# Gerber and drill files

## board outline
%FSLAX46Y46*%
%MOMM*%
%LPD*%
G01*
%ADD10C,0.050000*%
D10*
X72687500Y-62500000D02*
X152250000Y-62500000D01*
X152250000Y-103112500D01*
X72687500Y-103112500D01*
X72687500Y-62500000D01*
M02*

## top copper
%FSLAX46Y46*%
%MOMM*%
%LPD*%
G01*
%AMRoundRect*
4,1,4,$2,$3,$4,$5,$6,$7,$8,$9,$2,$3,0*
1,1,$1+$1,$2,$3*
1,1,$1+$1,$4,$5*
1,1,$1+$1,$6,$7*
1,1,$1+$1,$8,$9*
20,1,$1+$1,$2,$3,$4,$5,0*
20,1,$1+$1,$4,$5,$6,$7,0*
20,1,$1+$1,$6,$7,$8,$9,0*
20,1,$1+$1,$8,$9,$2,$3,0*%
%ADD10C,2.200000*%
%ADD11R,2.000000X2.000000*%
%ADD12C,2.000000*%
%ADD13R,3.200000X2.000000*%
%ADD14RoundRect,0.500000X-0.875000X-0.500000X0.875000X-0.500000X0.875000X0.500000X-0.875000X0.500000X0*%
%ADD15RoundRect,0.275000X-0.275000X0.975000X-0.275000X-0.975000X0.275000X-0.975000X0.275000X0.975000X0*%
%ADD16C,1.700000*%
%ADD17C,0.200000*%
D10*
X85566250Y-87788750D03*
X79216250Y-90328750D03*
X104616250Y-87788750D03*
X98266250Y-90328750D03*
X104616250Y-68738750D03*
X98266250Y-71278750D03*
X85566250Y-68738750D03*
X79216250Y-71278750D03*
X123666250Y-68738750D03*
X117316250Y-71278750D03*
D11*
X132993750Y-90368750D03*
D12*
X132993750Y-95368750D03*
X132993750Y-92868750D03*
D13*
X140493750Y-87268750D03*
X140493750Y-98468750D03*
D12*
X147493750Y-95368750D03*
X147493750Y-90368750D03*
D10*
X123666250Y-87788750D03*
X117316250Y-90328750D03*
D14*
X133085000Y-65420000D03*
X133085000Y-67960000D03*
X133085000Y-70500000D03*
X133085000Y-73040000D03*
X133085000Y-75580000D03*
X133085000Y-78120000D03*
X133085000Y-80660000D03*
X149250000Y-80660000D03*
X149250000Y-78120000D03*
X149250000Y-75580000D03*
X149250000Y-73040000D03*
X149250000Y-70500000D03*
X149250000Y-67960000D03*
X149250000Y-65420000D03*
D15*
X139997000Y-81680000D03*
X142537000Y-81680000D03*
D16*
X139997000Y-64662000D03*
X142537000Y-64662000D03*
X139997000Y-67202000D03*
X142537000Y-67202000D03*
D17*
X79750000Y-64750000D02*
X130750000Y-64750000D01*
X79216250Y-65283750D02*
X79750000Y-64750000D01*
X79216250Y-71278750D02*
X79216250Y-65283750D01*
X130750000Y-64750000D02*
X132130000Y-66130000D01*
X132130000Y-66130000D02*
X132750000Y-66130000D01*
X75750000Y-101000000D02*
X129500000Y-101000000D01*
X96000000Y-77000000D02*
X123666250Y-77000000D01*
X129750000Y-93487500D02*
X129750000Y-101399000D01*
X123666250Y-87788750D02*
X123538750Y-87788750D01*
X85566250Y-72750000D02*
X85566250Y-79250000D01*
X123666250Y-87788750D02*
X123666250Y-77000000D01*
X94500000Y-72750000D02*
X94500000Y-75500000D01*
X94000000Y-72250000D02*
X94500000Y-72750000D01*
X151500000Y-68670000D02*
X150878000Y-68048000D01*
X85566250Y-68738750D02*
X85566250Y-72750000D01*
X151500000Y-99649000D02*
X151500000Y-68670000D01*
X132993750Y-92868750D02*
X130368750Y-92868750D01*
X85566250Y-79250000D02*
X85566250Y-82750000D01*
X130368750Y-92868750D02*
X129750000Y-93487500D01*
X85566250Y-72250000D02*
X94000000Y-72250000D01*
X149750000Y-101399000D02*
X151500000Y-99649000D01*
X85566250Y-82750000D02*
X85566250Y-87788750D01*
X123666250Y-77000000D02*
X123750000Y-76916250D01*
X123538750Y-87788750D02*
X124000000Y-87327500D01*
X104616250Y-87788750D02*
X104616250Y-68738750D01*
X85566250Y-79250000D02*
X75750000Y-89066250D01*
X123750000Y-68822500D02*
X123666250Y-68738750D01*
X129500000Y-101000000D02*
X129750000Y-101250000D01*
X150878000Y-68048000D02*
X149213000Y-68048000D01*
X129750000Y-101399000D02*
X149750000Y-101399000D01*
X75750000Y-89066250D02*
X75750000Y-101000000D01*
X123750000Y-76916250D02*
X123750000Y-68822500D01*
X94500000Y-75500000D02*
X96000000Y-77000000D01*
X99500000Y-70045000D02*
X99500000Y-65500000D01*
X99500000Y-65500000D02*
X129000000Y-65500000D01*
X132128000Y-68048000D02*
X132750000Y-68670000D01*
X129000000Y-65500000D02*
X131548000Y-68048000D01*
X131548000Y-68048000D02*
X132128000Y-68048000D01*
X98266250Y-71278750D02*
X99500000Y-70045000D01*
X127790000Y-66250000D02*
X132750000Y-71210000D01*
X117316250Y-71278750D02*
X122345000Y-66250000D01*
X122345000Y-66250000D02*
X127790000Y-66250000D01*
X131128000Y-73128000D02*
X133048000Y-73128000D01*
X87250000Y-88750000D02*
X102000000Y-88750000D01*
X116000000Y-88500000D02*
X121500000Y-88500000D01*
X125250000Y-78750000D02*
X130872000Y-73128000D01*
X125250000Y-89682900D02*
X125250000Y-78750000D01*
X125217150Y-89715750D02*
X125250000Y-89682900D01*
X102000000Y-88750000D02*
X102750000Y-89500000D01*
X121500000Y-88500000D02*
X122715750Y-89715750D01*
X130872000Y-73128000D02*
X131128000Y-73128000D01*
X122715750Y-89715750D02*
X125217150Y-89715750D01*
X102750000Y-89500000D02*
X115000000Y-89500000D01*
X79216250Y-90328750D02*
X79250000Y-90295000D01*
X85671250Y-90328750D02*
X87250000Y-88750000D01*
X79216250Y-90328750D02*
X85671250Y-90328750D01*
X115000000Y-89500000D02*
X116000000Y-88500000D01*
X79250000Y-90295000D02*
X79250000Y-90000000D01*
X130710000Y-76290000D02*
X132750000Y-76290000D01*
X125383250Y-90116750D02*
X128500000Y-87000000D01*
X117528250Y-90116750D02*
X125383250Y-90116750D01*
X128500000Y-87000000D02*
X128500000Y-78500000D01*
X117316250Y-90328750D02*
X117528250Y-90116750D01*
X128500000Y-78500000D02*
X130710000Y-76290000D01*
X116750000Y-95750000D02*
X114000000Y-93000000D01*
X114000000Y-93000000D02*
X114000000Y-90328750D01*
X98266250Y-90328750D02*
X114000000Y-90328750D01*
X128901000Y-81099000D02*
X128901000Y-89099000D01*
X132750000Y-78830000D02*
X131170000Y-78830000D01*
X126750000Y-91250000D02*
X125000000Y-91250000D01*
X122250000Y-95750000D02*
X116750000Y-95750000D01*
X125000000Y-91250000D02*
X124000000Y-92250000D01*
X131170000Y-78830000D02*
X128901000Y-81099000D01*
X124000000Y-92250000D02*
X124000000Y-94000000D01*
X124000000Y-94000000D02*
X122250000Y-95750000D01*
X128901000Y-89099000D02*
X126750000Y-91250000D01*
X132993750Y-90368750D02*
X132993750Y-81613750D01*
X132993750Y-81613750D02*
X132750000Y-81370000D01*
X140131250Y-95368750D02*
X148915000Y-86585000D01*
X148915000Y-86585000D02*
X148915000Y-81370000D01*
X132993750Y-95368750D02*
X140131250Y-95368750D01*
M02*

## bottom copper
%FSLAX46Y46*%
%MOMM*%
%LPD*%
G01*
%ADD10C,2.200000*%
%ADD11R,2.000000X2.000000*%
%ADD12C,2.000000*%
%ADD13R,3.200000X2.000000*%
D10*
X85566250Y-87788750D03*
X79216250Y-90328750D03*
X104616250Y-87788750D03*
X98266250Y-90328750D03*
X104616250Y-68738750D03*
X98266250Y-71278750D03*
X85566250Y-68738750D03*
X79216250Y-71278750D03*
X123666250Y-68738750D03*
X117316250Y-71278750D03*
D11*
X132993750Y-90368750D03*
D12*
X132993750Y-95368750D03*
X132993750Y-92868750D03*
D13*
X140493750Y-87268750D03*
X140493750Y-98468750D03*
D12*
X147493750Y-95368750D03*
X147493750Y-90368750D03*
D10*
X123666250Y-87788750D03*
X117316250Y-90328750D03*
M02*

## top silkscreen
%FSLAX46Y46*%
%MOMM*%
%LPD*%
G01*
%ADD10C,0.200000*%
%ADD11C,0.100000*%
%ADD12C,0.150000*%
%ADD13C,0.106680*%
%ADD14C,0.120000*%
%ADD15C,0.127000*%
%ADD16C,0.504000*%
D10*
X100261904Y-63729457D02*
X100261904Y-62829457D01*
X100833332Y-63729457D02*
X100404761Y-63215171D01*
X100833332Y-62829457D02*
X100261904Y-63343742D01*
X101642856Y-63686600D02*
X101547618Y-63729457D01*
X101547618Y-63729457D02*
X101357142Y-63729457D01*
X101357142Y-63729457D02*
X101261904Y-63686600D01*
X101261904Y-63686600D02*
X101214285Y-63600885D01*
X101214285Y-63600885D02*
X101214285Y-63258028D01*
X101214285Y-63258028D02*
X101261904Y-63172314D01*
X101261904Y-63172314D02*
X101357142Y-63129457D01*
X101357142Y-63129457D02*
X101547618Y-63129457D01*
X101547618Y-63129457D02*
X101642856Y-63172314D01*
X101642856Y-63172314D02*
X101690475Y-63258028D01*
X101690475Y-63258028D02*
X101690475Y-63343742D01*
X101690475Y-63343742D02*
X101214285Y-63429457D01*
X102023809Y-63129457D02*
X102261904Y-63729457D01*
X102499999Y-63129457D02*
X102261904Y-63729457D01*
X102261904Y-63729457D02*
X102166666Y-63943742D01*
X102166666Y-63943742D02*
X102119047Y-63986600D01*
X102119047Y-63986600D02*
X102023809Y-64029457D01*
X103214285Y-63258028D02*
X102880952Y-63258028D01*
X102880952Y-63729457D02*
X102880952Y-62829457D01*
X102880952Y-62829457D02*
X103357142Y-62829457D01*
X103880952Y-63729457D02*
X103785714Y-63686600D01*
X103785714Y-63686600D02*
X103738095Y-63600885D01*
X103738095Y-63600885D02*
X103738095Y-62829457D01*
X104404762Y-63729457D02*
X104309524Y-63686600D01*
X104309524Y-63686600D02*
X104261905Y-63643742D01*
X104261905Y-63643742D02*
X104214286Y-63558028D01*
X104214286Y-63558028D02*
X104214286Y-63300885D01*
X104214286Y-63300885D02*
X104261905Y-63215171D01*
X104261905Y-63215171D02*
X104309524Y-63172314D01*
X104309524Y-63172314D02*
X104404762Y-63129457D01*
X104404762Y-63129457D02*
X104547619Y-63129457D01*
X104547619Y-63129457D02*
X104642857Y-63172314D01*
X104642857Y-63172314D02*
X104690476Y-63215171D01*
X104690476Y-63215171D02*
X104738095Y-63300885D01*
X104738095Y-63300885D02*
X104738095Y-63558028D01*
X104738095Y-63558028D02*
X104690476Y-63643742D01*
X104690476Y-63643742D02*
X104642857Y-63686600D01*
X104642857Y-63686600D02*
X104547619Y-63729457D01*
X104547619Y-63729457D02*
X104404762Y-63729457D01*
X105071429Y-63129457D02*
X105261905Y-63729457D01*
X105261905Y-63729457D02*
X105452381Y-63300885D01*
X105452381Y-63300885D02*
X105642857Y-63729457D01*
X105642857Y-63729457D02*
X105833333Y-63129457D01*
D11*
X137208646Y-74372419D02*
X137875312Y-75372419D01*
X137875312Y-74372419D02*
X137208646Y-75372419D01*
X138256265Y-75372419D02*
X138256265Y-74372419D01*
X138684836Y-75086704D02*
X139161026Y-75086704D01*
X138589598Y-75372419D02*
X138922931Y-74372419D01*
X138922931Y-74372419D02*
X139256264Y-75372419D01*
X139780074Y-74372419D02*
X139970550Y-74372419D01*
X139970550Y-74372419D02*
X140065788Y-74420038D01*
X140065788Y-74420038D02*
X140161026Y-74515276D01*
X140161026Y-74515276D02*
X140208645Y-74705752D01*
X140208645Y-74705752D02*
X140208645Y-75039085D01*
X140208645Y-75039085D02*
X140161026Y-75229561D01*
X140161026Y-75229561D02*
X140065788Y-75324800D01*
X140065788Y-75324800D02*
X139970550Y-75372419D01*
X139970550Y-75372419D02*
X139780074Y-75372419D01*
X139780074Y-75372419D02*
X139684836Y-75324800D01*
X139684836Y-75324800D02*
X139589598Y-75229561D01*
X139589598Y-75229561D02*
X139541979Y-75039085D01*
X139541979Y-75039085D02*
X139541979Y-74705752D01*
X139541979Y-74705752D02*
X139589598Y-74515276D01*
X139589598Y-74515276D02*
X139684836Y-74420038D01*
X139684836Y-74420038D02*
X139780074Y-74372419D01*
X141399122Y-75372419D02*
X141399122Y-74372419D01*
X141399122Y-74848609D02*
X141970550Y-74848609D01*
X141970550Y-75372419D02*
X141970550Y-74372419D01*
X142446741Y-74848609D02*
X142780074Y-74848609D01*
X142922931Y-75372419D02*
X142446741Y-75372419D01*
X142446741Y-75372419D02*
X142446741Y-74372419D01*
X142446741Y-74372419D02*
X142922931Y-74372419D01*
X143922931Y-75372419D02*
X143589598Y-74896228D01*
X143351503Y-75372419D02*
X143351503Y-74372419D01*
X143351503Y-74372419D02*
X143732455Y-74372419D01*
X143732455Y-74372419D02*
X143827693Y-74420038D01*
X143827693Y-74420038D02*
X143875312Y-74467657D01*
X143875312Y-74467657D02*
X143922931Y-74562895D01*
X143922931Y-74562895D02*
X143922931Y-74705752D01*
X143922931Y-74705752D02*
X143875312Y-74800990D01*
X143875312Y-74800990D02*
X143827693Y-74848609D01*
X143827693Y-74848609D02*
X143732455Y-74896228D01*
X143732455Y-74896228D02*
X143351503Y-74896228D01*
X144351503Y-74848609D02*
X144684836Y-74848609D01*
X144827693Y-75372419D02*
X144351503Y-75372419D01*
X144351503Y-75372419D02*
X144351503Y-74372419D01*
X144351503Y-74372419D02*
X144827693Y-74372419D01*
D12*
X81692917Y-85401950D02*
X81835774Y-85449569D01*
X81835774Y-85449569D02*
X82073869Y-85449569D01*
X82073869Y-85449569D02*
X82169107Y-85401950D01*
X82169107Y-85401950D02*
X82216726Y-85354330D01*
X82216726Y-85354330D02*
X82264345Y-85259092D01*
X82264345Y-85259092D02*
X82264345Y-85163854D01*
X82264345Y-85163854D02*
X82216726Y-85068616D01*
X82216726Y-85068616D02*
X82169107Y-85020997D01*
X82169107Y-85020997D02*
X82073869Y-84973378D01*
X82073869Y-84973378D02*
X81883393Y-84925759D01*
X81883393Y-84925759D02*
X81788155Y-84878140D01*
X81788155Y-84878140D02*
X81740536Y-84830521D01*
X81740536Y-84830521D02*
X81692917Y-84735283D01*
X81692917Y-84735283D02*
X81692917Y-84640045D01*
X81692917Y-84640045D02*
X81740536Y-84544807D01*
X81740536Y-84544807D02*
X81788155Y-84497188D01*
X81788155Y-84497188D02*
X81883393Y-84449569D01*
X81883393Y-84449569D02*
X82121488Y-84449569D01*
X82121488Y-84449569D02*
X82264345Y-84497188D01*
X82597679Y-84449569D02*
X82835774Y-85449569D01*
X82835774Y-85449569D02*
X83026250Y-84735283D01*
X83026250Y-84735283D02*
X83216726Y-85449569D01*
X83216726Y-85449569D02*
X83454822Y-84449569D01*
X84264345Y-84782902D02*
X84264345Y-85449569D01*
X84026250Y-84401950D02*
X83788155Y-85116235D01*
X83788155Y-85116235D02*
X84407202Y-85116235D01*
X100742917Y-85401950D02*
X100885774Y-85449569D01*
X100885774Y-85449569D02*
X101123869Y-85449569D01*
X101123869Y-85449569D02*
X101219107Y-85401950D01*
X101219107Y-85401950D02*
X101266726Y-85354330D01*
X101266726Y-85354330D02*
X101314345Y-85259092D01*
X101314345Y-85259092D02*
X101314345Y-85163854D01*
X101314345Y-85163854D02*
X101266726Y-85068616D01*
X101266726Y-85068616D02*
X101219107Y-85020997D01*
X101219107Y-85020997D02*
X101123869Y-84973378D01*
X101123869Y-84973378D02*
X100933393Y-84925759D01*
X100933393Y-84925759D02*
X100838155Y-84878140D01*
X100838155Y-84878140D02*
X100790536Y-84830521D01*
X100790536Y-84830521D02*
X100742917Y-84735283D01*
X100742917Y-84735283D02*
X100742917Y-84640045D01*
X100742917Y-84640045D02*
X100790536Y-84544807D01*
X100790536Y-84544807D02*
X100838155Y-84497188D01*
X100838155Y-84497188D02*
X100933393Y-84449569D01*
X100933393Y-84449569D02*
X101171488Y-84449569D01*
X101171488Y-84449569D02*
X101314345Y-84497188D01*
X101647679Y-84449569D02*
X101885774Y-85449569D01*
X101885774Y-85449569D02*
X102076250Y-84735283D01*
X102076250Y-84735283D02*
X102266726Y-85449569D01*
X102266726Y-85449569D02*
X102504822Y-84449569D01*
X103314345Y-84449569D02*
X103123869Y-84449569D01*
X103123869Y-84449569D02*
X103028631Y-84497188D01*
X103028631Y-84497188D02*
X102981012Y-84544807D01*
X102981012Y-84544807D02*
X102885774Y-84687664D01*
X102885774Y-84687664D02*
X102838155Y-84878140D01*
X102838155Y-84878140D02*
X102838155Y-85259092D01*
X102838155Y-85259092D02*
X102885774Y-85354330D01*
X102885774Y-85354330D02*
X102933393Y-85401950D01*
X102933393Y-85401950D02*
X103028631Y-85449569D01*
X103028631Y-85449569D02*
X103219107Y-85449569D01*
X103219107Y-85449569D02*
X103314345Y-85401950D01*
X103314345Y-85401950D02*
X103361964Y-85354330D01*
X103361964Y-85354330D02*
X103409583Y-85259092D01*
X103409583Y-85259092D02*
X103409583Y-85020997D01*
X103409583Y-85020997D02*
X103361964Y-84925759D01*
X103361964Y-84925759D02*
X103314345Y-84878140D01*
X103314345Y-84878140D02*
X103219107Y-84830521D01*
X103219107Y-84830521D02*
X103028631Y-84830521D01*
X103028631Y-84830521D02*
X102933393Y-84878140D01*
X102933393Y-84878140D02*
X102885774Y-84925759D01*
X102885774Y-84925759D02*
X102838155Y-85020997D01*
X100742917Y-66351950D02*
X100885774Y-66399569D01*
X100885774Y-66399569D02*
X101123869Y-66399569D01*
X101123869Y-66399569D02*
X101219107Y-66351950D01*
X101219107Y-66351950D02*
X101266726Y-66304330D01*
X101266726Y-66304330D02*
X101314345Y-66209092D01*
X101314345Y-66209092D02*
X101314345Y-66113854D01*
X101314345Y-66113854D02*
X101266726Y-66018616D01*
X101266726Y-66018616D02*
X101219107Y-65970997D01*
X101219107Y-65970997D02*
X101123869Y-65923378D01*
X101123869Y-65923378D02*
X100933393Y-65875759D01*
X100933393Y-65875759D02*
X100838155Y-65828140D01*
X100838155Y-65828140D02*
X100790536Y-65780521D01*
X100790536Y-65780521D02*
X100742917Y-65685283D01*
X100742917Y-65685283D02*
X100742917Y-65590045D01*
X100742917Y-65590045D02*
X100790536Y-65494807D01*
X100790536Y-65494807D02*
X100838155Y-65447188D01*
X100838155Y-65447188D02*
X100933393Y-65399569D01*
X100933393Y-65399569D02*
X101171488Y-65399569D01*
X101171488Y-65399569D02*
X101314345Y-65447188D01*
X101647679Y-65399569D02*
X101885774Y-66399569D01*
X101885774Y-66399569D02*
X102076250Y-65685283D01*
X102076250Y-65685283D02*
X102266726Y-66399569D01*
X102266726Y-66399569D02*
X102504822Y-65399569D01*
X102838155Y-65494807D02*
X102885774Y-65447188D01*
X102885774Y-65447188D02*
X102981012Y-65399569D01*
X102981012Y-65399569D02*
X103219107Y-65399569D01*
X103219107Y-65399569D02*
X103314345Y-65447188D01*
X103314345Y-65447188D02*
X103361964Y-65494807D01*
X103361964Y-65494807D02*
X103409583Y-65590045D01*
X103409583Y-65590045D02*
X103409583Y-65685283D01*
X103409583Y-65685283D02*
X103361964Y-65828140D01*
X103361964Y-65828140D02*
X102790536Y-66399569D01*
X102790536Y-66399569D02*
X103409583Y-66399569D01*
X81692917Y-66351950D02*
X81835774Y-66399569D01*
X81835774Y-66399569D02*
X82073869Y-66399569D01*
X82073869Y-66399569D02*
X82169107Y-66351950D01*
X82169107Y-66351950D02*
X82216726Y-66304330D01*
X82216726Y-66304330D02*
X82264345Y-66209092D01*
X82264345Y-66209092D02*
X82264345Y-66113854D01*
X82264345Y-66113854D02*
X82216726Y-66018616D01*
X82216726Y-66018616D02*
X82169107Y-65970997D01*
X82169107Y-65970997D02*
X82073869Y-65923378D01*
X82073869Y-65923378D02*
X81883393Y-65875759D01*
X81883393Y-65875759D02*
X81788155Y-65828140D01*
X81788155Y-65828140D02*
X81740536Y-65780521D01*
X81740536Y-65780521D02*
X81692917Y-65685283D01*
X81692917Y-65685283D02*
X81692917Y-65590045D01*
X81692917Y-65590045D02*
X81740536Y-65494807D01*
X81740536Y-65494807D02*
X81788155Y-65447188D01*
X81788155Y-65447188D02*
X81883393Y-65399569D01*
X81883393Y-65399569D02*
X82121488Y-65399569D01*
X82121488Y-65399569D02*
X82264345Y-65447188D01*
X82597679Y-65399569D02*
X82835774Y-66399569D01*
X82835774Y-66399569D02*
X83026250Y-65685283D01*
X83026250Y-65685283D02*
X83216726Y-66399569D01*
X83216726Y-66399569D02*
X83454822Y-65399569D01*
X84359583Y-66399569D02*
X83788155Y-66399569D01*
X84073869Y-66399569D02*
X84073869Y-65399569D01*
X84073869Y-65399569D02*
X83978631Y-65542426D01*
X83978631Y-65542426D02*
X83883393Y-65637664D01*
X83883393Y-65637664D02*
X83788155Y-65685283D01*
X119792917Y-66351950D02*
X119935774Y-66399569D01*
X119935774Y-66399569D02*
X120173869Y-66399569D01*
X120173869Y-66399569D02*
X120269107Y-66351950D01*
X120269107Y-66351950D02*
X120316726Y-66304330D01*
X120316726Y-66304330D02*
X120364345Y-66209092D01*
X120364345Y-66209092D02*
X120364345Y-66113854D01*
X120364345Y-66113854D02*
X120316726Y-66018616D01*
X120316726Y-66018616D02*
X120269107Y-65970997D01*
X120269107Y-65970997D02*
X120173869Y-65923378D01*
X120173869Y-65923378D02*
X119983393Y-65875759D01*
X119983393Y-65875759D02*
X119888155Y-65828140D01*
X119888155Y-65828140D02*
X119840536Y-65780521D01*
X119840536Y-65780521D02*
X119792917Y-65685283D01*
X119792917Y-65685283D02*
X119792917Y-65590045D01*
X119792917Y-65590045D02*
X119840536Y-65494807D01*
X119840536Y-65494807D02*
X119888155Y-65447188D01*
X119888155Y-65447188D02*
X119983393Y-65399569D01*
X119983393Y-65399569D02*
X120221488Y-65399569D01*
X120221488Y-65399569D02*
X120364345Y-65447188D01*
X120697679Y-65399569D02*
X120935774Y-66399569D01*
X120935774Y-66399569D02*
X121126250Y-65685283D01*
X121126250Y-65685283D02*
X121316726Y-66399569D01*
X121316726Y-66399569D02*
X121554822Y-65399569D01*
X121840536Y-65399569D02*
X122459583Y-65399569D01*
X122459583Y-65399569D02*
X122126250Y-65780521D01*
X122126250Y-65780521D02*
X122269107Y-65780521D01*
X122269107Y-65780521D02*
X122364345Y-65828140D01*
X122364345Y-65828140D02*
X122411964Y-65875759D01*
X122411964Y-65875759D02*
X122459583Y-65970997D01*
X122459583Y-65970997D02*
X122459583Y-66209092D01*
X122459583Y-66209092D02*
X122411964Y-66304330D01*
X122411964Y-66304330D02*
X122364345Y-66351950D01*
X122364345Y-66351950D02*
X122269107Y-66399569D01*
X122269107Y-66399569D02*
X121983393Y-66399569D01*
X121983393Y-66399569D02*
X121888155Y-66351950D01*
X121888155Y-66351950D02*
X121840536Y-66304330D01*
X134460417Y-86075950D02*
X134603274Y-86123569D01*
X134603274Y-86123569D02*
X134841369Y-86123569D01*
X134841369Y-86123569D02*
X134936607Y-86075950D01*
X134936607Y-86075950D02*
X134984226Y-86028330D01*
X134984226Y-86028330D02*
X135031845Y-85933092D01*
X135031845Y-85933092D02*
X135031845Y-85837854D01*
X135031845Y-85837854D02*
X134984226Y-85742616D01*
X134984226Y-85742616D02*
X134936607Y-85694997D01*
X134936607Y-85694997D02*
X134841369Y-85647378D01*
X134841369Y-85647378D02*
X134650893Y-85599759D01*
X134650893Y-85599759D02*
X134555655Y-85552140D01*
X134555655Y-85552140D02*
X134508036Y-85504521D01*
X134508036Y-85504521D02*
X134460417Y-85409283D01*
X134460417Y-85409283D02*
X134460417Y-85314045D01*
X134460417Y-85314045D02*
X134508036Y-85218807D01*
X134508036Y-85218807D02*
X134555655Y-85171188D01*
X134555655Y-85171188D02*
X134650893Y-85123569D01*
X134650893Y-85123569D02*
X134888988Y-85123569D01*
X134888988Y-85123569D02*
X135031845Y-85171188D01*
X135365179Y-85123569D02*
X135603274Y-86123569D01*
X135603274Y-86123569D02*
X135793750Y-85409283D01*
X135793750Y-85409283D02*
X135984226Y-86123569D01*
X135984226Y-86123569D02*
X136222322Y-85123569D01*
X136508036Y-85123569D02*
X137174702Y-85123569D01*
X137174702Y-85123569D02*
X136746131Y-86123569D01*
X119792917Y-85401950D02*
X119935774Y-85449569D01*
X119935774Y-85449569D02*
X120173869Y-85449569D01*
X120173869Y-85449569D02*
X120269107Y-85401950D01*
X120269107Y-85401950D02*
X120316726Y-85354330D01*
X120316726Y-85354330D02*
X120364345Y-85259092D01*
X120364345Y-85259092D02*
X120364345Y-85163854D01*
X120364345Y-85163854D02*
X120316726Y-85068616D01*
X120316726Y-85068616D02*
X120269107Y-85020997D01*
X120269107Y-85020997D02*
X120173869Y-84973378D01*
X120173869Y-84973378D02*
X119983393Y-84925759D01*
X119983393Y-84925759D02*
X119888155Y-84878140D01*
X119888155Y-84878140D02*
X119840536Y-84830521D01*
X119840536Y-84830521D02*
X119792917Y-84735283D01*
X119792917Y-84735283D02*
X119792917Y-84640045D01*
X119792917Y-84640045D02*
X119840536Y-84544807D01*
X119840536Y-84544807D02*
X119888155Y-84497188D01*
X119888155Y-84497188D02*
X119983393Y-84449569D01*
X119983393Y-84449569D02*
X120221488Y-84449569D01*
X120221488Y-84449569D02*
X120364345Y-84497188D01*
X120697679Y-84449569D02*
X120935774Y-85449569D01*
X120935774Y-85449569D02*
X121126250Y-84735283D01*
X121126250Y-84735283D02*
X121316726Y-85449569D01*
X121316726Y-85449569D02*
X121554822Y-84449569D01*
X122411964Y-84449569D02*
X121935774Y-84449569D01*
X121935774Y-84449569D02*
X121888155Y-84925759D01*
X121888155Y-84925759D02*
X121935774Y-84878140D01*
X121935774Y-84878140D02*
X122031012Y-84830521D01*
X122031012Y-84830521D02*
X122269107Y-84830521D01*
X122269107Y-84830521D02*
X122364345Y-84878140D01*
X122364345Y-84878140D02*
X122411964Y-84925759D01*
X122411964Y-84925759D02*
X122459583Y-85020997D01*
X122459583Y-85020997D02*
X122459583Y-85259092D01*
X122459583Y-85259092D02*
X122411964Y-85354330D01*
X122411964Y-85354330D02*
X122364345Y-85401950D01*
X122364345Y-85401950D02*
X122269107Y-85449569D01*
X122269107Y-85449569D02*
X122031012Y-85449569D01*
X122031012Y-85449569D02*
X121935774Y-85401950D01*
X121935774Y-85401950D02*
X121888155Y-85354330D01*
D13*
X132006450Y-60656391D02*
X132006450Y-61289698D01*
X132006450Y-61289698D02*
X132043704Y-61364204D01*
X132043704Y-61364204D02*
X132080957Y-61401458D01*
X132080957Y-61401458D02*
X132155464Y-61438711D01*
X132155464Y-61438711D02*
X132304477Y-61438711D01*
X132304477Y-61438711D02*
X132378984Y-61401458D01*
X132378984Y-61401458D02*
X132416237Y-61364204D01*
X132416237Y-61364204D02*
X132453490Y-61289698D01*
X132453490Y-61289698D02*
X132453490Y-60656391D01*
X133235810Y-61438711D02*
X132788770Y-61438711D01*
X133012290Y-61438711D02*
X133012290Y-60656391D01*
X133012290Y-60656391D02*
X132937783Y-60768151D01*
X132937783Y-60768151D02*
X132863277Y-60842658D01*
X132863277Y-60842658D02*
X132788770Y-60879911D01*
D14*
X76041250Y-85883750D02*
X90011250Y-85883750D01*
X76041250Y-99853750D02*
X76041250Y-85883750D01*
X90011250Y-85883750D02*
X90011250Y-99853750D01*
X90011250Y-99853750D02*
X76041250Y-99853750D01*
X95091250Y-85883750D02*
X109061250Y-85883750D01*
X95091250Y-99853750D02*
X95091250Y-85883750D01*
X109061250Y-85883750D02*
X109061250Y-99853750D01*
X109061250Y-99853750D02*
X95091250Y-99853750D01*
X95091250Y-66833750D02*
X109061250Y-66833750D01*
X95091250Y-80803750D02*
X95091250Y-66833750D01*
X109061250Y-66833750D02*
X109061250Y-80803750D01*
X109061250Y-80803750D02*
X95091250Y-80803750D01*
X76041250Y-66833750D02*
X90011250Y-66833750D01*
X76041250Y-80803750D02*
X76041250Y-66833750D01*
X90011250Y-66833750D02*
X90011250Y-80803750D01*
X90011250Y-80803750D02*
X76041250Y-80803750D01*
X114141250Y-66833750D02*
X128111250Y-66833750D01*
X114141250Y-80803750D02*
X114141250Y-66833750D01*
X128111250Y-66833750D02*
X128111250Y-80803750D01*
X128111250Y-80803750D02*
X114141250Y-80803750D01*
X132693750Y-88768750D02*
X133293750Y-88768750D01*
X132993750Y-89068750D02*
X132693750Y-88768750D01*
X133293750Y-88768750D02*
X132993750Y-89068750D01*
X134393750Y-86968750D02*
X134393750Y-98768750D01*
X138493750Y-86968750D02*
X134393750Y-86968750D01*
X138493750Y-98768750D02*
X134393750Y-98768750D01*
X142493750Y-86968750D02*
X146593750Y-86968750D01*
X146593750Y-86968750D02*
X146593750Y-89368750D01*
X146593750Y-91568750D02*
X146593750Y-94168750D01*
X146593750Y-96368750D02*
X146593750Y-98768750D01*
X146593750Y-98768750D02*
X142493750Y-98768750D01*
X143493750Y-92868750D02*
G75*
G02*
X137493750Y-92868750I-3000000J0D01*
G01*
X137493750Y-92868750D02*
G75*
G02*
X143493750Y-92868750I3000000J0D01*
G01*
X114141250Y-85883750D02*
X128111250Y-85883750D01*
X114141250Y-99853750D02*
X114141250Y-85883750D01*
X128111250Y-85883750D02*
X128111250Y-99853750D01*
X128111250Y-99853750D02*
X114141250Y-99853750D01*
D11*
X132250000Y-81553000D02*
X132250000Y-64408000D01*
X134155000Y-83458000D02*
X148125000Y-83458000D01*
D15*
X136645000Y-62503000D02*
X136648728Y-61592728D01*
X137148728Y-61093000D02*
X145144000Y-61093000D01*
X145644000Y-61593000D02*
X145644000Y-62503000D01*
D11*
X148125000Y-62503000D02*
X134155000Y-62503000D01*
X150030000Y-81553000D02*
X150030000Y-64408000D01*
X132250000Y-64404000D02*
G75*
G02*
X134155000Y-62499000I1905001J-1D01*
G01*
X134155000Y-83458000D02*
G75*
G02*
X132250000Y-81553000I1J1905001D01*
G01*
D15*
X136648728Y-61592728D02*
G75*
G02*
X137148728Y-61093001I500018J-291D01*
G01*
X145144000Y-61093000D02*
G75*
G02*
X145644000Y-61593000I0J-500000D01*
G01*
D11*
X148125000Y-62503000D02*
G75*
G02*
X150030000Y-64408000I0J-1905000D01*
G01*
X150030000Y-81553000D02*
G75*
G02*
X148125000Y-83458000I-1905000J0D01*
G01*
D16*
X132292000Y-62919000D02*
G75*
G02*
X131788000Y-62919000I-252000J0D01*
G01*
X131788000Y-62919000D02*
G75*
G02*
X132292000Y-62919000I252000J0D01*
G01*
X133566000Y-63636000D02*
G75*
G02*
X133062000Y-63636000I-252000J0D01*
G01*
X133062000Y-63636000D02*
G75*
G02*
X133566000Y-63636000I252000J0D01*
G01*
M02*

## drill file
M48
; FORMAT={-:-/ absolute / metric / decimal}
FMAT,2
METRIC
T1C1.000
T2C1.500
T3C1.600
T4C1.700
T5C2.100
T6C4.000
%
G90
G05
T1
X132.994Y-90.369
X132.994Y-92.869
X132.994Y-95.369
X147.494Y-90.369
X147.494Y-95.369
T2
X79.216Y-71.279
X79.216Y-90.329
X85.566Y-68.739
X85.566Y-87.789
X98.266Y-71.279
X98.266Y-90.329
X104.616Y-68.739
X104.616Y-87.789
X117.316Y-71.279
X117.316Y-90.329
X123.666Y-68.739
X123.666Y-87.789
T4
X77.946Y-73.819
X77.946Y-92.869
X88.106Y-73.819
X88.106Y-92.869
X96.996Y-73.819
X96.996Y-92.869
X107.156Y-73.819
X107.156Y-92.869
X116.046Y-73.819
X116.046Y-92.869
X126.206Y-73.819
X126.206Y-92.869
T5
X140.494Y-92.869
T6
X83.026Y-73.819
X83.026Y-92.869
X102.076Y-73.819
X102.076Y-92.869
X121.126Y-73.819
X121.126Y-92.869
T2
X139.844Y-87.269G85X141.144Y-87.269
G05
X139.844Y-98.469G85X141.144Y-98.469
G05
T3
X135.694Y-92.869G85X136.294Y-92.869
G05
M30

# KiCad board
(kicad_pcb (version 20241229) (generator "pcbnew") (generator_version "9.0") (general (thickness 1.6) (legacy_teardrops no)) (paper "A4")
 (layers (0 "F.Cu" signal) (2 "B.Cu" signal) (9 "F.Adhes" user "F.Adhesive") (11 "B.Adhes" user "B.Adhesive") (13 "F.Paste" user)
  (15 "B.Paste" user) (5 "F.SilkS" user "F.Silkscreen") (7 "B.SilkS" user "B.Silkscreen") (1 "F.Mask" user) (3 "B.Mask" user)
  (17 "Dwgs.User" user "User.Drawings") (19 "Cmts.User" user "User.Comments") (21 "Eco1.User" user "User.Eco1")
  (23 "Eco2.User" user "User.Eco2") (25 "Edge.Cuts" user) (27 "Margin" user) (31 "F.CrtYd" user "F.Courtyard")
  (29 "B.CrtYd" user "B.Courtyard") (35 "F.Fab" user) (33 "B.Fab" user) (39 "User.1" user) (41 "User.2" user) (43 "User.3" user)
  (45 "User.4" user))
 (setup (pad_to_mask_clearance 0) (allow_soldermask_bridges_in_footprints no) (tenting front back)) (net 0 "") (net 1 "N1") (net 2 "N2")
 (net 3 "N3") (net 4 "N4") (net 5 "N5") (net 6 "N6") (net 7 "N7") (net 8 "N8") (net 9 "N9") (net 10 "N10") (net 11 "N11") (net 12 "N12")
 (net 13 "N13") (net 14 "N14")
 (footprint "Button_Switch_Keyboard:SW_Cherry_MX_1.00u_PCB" (layer "F.Cu") (at 85.56625 87.78875)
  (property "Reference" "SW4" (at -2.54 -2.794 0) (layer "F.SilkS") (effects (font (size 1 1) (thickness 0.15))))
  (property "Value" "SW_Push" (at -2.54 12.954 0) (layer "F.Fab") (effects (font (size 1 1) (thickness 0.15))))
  (fp_line (start -9.525 -1.905) (end 4.445 -1.905) (stroke (width 0.12) (type solid)) (layer "F.SilkS"))
  (fp_line (start -9.525 12.065) (end -9.525 -1.905) (stroke (width 0.12) (type solid)) (layer "F.SilkS"))
  (fp_line (start 4.445 -1.905) (end 4.445 12.065) (stroke (width 0.12) (type solid)) (layer "F.SilkS"))
  (fp_line (start 4.445 12.065) (end -9.525 12.065) (stroke (width 0.12) (type solid)) (layer "F.SilkS"))
  (pad "" np_thru_hole circle (at -7.62 5.08) (size 1.7 1.7) (drill 1.7) (layers "*.Cu" "*.Mask"))
  (pad "" np_thru_hole circle (at -2.54 5.08) (size 4 4) (drill 4) (layers "*.Cu" "*.Mask"))
  (pad "" np_thru_hole circle (at 2.54 5.08) (size 1.7 1.7) (drill 1.7) (layers "*.Cu" "*.Mask"))
  (pad "1" thru_hole circle (at 0 0) (size 2.2 2.2) (drill 1.5) (layers "*.Cu" "*.Mask") (remove_unused_layers no) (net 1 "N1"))
  (pad "2" thru_hole circle (at -6.35 2.54) (size 2.2 2.2) (drill 1.5) (layers "*.Cu" "*.Mask") (remove_unused_layers no) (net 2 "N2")))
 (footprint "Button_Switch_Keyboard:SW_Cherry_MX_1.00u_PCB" (layer "F.Cu") (at 104.61625 87.78875)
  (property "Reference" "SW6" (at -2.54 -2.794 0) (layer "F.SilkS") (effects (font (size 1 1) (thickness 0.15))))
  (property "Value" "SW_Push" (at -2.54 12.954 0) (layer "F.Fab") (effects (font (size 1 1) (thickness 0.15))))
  (fp_line (start -9.525 -1.905) (end 4.445 -1.905) (stroke (width 0.12) (type solid)) (layer "F.SilkS"))
  (fp_line (start -9.525 12.065) (end -9.525 -1.905) (stroke (width 0.12) (type solid)) (layer "F.SilkS"))
  (fp_line (start 4.445 -1.905) (end 4.445 12.065) (stroke (width 0.12) (type solid)) (layer "F.SilkS"))
  (fp_line (start 4.445 12.065) (end -9.525 12.065) (stroke (width 0.12) (type solid)) (layer "F.SilkS"))
  (pad "" np_thru_hole circle (at -7.62 5.08) (size 1.7 1.7) (drill 1.7) (layers "*.Cu" "*.Mask"))
  (pad "" np_thru_hole circle (at -2.54 5.08) (size 4 4) (drill 4) (layers "*.Cu" "*.Mask"))
  (pad "" np_thru_hole circle (at 2.54 5.08) (size 1.7 1.7) (drill 1.7) (layers "*.Cu" "*.Mask"))
  (pad "1" thru_hole circle (at 0 0) (size 2.2 2.2) (drill 1.5) (layers "*.Cu" "*.Mask") (remove_unused_layers no) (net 1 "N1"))
  (pad "2" thru_hole circle (at -6.35 2.54) (size 2.2 2.2) (drill 1.5) (layers "*.Cu" "*.Mask") (remove_unused_layers no) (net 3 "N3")))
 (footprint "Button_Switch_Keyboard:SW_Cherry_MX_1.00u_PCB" (layer "F.Cu") (at 104.61625 68.73875)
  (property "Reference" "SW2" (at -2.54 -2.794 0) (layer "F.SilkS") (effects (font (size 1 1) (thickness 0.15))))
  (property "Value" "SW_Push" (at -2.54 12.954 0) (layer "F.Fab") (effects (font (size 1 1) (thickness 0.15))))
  (fp_line (start -9.525 -1.905) (end 4.445 -1.905) (stroke (width 0.12) (type solid)) (layer "F.SilkS"))
  (fp_line (start -9.525 12.065) (end -9.525 -1.905) (stroke (width 0.12) (type solid)) (layer "F.SilkS"))
  (fp_line (start 4.445 -1.905) (end 4.445 12.065) (stroke (width 0.12) (type solid)) (layer "F.SilkS"))
  (fp_line (start 4.445 12.065) (end -9.525 12.065) (stroke (width 0.12) (type solid)) (layer "F.SilkS"))
  (pad "" np_thru_hole circle (at -7.62 5.08) (size 1.7 1.7) (drill 1.7) (layers "*.Cu" "*.Mask"))
  (pad "" np_thru_hole circle (at -2.54 5.08) (size 4 4) (drill 4) (layers "*.Cu" "*.Mask"))
  (pad "" np_thru_hole circle (at 2.54 5.08) (size 1.7 1.7) (drill 1.7) (layers "*.Cu" "*.Mask"))
  (pad "1" thru_hole circle (at 0 0) (size 2.2 2.2) (drill 1.5) (layers "*.Cu" "*.Mask") (remove_unused_layers no) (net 1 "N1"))
  (pad "2" thru_hole circle (at -6.35 2.54) (size 2.2 2.2) (drill 1.5) (layers "*.Cu" "*.Mask") (remove_unused_layers no) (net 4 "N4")))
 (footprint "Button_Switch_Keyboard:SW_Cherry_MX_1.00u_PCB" (layer "F.Cu") (at 85.56625 68.73875)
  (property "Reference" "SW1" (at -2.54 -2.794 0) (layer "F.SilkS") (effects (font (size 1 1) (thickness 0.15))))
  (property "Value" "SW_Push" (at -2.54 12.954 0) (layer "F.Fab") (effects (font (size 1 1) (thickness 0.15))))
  (fp_line (start -9.525 -1.905) (end 4.445 -1.905) (stroke (width 0.12) (type solid)) (layer "F.SilkS"))
  (fp_line (start -9.525 12.065) (end -9.525 -1.905) (stroke (width 0.12) (type solid)) (layer "F.SilkS"))
  (fp_line (start 4.445 -1.905) (end 4.445 12.065) (stroke (width 0.12) (type solid)) (layer "F.SilkS"))
  (fp_line (start 4.445 12.065) (end -9.525 12.065) (stroke (width 0.12) (type solid)) (layer "F.SilkS"))
  (pad "" np_thru_hole circle (at -7.62 5.08) (size 1.7 1.7) (drill 1.7) (layers "*.Cu" "*.Mask"))
  (pad "" np_thru_hole circle (at -2.54 5.08) (size 4 4) (drill 4) (layers "*.Cu" "*.Mask"))
  (pad "" np_thru_hole circle (at 2.54 5.08) (size 1.7 1.7) (drill 1.7) (layers "*.Cu" "*.Mask"))
  (pad "1" thru_hole circle (at 0 0) (size 2.2 2.2) (drill 1.5) (layers "*.Cu" "*.Mask") (remove_unused_layers no) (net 1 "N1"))
  (pad "2" thru_hole circle (at -6.35 2.54) (size 2.2 2.2) (drill 1.5) (layers "*.Cu" "*.Mask") (remove_unused_layers no) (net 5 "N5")))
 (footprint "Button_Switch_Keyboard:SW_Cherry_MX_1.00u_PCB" (layer "F.Cu") (at 123.66625 68.73875)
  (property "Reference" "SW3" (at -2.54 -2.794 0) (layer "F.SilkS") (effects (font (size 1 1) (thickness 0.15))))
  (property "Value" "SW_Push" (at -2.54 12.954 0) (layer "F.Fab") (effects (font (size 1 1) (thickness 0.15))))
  (fp_line (start -9.525 -1.905) (end 4.445 -1.905) (stroke (width 0.12) (type solid)) (layer "F.SilkS"))
  (fp_line (start -9.525 12.065) (end -9.525 -1.905) (stroke (width 0.12) (type solid)) (layer "F.SilkS"))
  (fp_line (start 4.445 -1.905) (end 4.445 12.065) (stroke (width 0.12) (type solid)) (layer "F.SilkS"))
  (fp_line (start 4.445 12.065) (end -9.525 12.065) (stroke (width 0.12) (type solid)) (layer "F.SilkS"))
  (pad "" np_thru_hole circle (at -7.62 5.08) (size 1.7 1.7) (drill 1.7) (layers "*.Cu" "*.Mask"))
  (pad "" np_thru_hole circle (at -2.54 5.08) (size 4 4) (drill 4) (layers "*.Cu" "*.Mask"))
  (pad "" np_thru_hole circle (at 2.54 5.08) (size 1.7 1.7) (drill 1.7) (layers "*.Cu" "*.Mask"))
  (pad "1" thru_hole circle (at 0 0) (size 2.2 2.2) (drill 1.5) (layers "*.Cu" "*.Mask") (remove_unused_layers no) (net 1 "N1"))
  (pad "2" thru_hole circle (at -6.35 2.54) (size 2.2 2.2) (drill 1.5) (layers "*.Cu" "*.Mask") (remove_unused_layers no) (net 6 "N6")))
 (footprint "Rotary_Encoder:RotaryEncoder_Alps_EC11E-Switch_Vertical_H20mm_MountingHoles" (layer "F.Cu") (at 132.99375 90.36875)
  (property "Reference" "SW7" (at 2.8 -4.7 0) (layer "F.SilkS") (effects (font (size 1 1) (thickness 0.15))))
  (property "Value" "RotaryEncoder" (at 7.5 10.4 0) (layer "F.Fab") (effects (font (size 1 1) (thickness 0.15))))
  (fp_line (start -0.3 -1.6) (end 0.3 -1.6) (stroke (width 0.12) (type solid)) (layer "F.SilkS"))
  (fp_line (start 0 -1.3) (end -0.3 -1.6) (stroke (width 0.12) (type solid)) (layer "F.SilkS"))
  (fp_line (start 0.3 -1.6) (end 0 -1.3) (stroke (width 0.12) (type solid)) (layer "F.SilkS"))
  (fp_line (start 1.4 -3.4) (end 1.4 8.4) (stroke (width 0.12) (type solid)) (layer "F.SilkS"))
  (fp_line (start 5.5 -3.4) (end 1.4 -3.4) (stroke (width 0.12) (type solid)) (layer "F.SilkS"))
  (fp_line (start 5.5 8.4) (end 1.4 8.4) (stroke (width 0.12) (type solid)) (layer "F.SilkS"))
  (fp_line (start 9.5 -3.4) (end 13.6 -3.4) (stroke (width 0.12) (type solid)) (layer "F.SilkS"))
  (fp_line (start 13.6 -3.4) (end 13.6 -1) (stroke (width 0.12) (type solid)) (layer "F.SilkS"))
  (fp_line (start 13.6 1.2) (end 13.6 3.8) (stroke (width 0.12) (type solid)) (layer "F.SilkS"))
  (fp_line (start 13.6 6) (end 13.6 8.4) (stroke (width 0.12) (type solid)) (layer "F.SilkS"))
  (fp_line (start 13.6 8.4) (end 9.5 8.4) (stroke (width 0.12) (type solid)) (layer "F.SilkS"))
  (fp_circle (center 7.5 2.5) (end 10.5 2.5) (stroke (width 0.12) (type solid)) (fill no) (layer "F.SilkS"))
  (pad "" np_thru_hole oval (at 3 2.5) (size 2.2 1.6) (drill oval 2.2 1.6) (layers "*.Mask"))
  (pad "" np_thru_hole circle (at 7.5 2.5) (size 2.1 2.1) (drill 2.1) (layers "*.Mask"))
  (pad "A" thru_hole rect (at 0 0) (size 2 2) (drill 1) (layers "*.Cu" "*.Mask") (remove_unused_layers no) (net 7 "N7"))
  (pad "B" thru_hole circle (at 0 5) (size 2 2) (drill 1) (layers "*.Cu" "*.Mask") (remove_unused_layers no) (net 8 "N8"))
  (pad "C" thru_hole circle (at 0 2.5) (size 2 2) (drill 1) (layers "*.Cu" "*.Mask") (remove_unused_layers no) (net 1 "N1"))
  (pad "MP" thru_hole rect (at 7.5 -3.1) (size 3.2 2) (drill oval 2.8 1.5) (layers "*.Cu" "*.Mask") (remove_unused_layers no))
  (pad "MP" thru_hole rect (at 7.5 8.1) (size 3.2 2) (drill oval 2.8 1.5) (layers "*.Cu" "*.Mask") (remove_unused_layers no))
  (pad "S1" thru_hole circle (at 14.5 5) (size 2 2) (drill 1) (layers "*.Cu" "*.Mask") (remove_unused_layers no))
  (pad "S2" thru_hole circle (at 14.5 0) (size 2 2) (drill 1) (layers "*.Cu" "*.Mask") (remove_unused_layers no)))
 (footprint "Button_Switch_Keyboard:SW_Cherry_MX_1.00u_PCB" (layer "F.Cu") (at 123.66625 87.78875)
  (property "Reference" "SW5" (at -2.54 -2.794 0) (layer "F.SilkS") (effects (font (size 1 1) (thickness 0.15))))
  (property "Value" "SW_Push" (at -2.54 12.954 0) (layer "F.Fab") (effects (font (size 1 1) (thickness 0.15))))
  (fp_line (start -9.525 -1.905) (end 4.445 -1.905) (stroke (width 0.12) (type solid)) (layer "F.SilkS"))
  (fp_line (start -9.525 12.065) (end -9.525 -1.905) (stroke (width 0.12) (type solid)) (layer "F.SilkS"))
  (fp_line (start 4.445 -1.905) (end 4.445 12.065) (stroke (width 0.12) (type solid)) (layer "F.SilkS"))
  (fp_line (start 4.445 12.065) (end -9.525 12.065) (stroke (width 0.12) (type solid)) (layer "F.SilkS"))
  (pad "" np_thru_hole circle (at -7.62 5.08) (size 1.7 1.7) (drill 1.7) (layers "*.Cu" "*.Mask"))
  (pad "" np_thru_hole circle (at -2.54 5.08) (size 4 4) (drill 4) (layers "*.Cu" "*.Mask"))
  (pad "" np_thru_hole circle (at 2.54 5.08) (size 1.7 1.7) (drill 1.7) (layers "*.Cu" "*.Mask"))
  (pad "1" thru_hole circle (at 0 0) (size 2.2 2.2) (drill 1.5) (layers "*.Cu" "*.Mask") (remove_unused_layers no) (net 1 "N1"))
  (pad "2" thru_hole circle (at -6.35 2.54) (size 2.2 2.2) (drill 1.5) (layers "*.Cu" "*.Mask") (remove_unused_layers no) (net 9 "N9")))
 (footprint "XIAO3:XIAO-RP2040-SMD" (layer "F.Cu") (at 141.085 73.04)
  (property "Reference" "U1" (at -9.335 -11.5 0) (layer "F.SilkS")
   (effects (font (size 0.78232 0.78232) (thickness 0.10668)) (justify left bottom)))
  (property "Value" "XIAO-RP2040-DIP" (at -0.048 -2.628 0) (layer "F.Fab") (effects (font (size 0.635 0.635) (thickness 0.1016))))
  (fp_line (start -8.835 8.513) (end -8.835 -8.632) (stroke (width 0.1) (type solid)) (layer "F.SilkS"))
  (fp_line (start -6.93 10.418) (end 7.04 10.418) (stroke (width 0.1) (type solid)) (layer "F.SilkS"))
  (fp_line (start -4.44 -10.537) (end -4.436272 -11.447272) (stroke (width 0.127) (type solid)) (layer "F.SilkS"))
  (fp_line (start -3.936272 -11.947) (end 4.059 -11.947) (stroke (width 0.127) (type solid)) (layer "F.SilkS"))
  (fp_line (start 4.559 -11.447) (end 4.559 -10.537) (stroke (width 0.127) (type solid)) (layer "F.SilkS"))
  (fp_line (start 7.04 -10.537) (end -6.93 -10.537) (stroke (width 0.1) (type solid)) (layer "F.SilkS"))
  (fp_line (start 8.945 8.513) (end 8.945 -8.632) (stroke (width 0.1) (type solid)) (layer "F.SilkS"))
  (fp_arc (start -8.835 -8.636) (mid -8.277038 -9.983038) (end -6.93 -10.541) (stroke (width 0.1) (type solid)) (layer "F.SilkS"))
  (fp_arc (start -6.93 10.418) (mid -8.277038 9.860038) (end -8.835 8.513) (stroke (width 0.1) (type solid)) (layer "F.SilkS"))
  (fp_arc (start -4.436272 -11.447272) (mid -4.289724 -11.800644) (end -3.936272 -11.947) (stroke (width 0.127) (type default))
   (layer "F.SilkS"))
  (fp_arc (start 4.059 -11.947) (mid 4.412553 -11.800553) (end 4.559 -11.447) (stroke (width 0.127) (type default)) (layer "F.SilkS"))
  (fp_arc (start 7.04 -10.537) (mid 8.387038 -9.979038) (end 8.945 -8.632) (stroke (width 0.1) (type solid)) (layer "F.SilkS"))
  (fp_arc (start 8.945 8.513) (mid 8.387038 9.860038) (end 7.04 10.418) (stroke (width 0.1) (type solid)) (layer "F.SilkS"))
  (fp_circle (center -9.045 -10.121) (end -9.045 -10.375) (stroke (width 0.5) (type solid)) (fill yes) (layer "F.SilkS"))
  (fp_circle (center -7.771 -9.404) (end -7.771 -9.658) (stroke (width 0.5) (type solid)) (fill yes) (layer "F.SilkS"))
  (pad "1" smd roundrect (at -8 -7.62) (size 2.75 2) (layers "F.Cu" "F.Mask" "F.Paste") (roundrect_rratio 0.25) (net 5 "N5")
   (solder_mask_margin 0.0508) (thermal_bridge_angle 45))
  (pad "2" smd roundrect (at -8 -5.08) (size 2.75 2) (layers "F.Cu" "F.Mask" "F.Paste") (roundrect_rratio 0.25) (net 4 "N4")
   (solder_mask_margin 0.0508) (thermal_bridge_angle 45))
  (pad "3" smd roundrect (at -8 -2.54) (size 2.75 2) (layers "F.Cu" "F.Mask" "F.Paste") (roundrect_rratio 0.25) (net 6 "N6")
   (solder_mask_margin 0.0508) (thermal_bridge_angle 45))
  (pad "4" smd roundrect (at -8 0) (size 2.75 2) (layers "F.Cu" "F.Mask" "F.Paste") (roundrect_rratio 0.25) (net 2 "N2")
   (solder_mask_margin 0.0508) (thermal_bridge_angle 45))
  (pad "5" smd roundrect (at -8 2.54) (size 2.75 2) (layers "F.Cu" "F.Mask" "F.Paste") (roundrect_rratio 0.25) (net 9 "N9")
   (solder_mask_margin 0.0508) (thermal_bridge_angle 45))
  (pad "6" smd roundrect (at -8 5.08) (size 2.75 2) (layers "F.Cu" "F.Mask" "F.Paste") (roundrect_rratio 0.25) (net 3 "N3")
   (solder_mask_margin 0.0508) (thermal_bridge_angle 45))
  (pad "7" smd roundrect (at -8 7.62) (size 2.75 2) (layers "F.Cu" "F.Mask" "F.Paste") (roundrect_rratio 0.25) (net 7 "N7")
   (solder_mask_margin 0.0508) (thermal_bridge_angle 45))
  (pad "8" smd roundrect (at 8.165 7.62) (size 2.75 2) (layers "F.Cu" "F.Mask" "F.Paste") (roundrect_rratio 0.25) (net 8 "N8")
   (solder_mask_margin 0.0508) (thermal_bridge_angle 45))
  (pad "9" smd roundrect (at 8.165 5.08) (size 2.75 2) (layers "F.Cu" "F.Mask" "F.Paste") (roundrect_rratio 0.25) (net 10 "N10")
   (solder_mask_margin 0.0508) (thermal_bridge_angle 45))
  (pad "10" smd roundrect (at 8.165 2.54) (size 2.75 2) (layers "F.Cu" "F.Mask" "F.Paste") (roundrect_rratio 0.25) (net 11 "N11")
   (solder_mask_margin 0.0508) (thermal_bridge_angle 45))
  (pad "11" smd roundrect (at 8.165 0) (size 2.75 2) (layers "F.Cu" "F.Mask" "F.Paste") (roundrect_rratio 0.25) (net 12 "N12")
   (solder_mask_margin 0.0508) (thermal_bridge_angle 45))
  (pad "12" smd roundrect (at 8.165 -2.54) (size 2.75 2) (layers "F.Cu" "F.Mask" "F.Paste") (roundrect_rratio 0.25) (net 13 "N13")
   (solder_mask_margin 0.0508) (thermal_bridge_angle 45))
  (pad "13" smd roundrect (at 8.165 -5.08) (size 2.75 2) (layers "F.Cu" "F.Mask" "F.Paste") (roundrect_rratio 0.25) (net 1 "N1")
   (solder_mask_margin 0.0508) (thermal_bridge_angle 45))
  (pad "14" smd roundrect (at 8.165 -7.62) (size 2.75 2) (layers "F.Cu" "F.Mask" "F.Paste") (roundrect_rratio 0.25) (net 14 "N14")
   (solder_mask_margin 0.0508) (thermal_bridge_angle 45))
  (pad "15" smd roundrect (at -1.088 8.64 270) (size 2.5 1.1) (layers "F.Cu" "F.Mask" "F.Paste") (roundrect_rratio 0.25)
   (thermal_bridge_angle 45))
  (pad "16" smd roundrect (at 1.452 8.64 270) (size 2.5 1.1) (layers "F.Cu" "F.Mask" "F.Paste") (roundrect_rratio 0.25)
   (thermal_bridge_angle 45))
  (pad "17" smd circle (at -1.088 -8.378) (size 1.7 1.7) (layers "F.Cu" "F.Mask" "F.Paste"))
  (pad "18" smd circle (at 1.452 -8.378) (size 1.7 1.7) (layers "F.Cu" "F.Mask" "F.Paste"))
  (pad "19" smd circle (at -1.088 -5.838) (size 1.7 1.7) (layers "F.Cu" "F.Mask" "F.Paste"))
  (pad "20" smd circle (at 1.452 -5.838) (size 1.7 1.7) (layers "F.Cu" "F.Mask" "F.Paste")))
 (gr_rect (start 72.6875 62.5) (end 152.25 103.1125) (stroke (width 0.05) (type default)) (fill no) (layer "Edge.Cuts"))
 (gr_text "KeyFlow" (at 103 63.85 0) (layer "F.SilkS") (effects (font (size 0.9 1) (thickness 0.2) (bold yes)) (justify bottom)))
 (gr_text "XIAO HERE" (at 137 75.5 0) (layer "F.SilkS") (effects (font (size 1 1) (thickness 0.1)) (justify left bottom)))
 (segment (start 79.75 64.75) (end 130.75 64.75) (width 0.2) (layer "F.Cu") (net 5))
 (segment (start 79.21625 65.28375) (end 79.75 64.75) (width 0.2) (layer "F.Cu") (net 5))
 (segment (start 79.21625 71.27875) (end 79.21625 65.28375) (width 0.2) (layer "F.Cu") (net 5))
 (segment (start 130.75 64.75) (end 132.13 66.13) (width 0.2) (layer "F.Cu") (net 5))
 (segment (start 132.13 66.13) (end 132.75 66.13) (width 0.2) (layer "F.Cu") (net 5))
 (segment (start 75.75 101) (end 129.5 101) (width 0.2) (layer "F.Cu") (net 1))
 (segment (start 96 77) (end 123.66625 77) (width 0.2) (layer "F.Cu") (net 1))
 (segment (start 129.75 93.4875) (end 129.75 101.399) (width 0.2) (layer "F.Cu") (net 1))
 (segment (start 123.66625 87.78875) (end 123.53875 87.78875) (width 0.2) (layer "F.Cu") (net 1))
 (segment (start 85.56625 72.75) (end 85.56625 79.25) (width 0.2) (layer "F.Cu") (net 1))
 (segment (start 123.66625 87.78875) (end 123.66625 77) (width 0.2) (layer "F.Cu") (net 1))
 (segment (start 94.5 72.75) (end 94.5 75.5) (width 0.2) (layer "F.Cu") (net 1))
 (segment (start 94 72.25) (end 94.5 72.75) (width 0.2) (layer "F.Cu") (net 1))
 (segment (start 151.5 68.67) (end 150.878 68.048) (width 0.2) (layer "F.Cu") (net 1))
 (segment (start 85.56625 68.73875) (end 85.56625 72.75) (width 0.2) (layer "F.Cu") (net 1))
 (segment (start 151.5 99.649) (end 151.5 68.67) (width 0.2) (layer "F.Cu") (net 1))
 (segment (start 132.99375 92.86875) (end 130.36875 92.86875) (width 0.2) (layer "F.Cu") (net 1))
 (segment (start 85.56625 79.25) (end 85.56625 82.75) (width 0.2) (layer "F.Cu") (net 1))
 (segment (start 130.36875 92.86875) (end 129.75 93.4875) (width 0.2) (layer "F.Cu") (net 1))
 (segment (start 85.56625 72.25) (end 94 72.25) (width 0.2) (layer "F.Cu") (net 1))
 (segment (start 149.75 101.399) (end 151.5 99.649) (width 0.2) (layer "F.Cu") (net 1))
 (segment (start 85.56625 82.75) (end 85.56625 87.78875) (width 0.2) (layer "F.Cu") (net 1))
 (segment (start 123.66625 77) (end 123.75 76.91625) (width 0.2) (layer "F.Cu") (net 1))
 (segment (start 123.53875 87.78875) (end 124 87.3275) (width 0.2) (layer "F.Cu") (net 1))
 (segment (start 104.61625 87.78875) (end 104.61625 68.73875) (width 0.2) (layer "F.Cu") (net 1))
 (segment (start 85.56625 79.25) (end 75.75 89.06625) (width 0.2) (layer "F.Cu") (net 1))
 (segment (start 123.75 68.8225) (end 123.66625 68.73875) (width 0.2) (layer "F.Cu") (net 1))
 (segment (start 129.5 101) (end 129.75 101.25) (width 0.2) (layer "F.Cu") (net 1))
 (segment (start 150.878 68.048) (end 149.213 68.048) (width 0.2) (layer "F.Cu") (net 1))
 (segment (start 129.75 101.399) (end 149.75 101.399) (width 0.2) (layer "F.Cu") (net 1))
 (segment (start 75.75 89.06625) (end 75.75 101) (width 0.2) (layer "F.Cu") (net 1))
 (segment (start 123.75 76.91625) (end 123.75 68.8225) (width 0.2) (layer "F.Cu") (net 1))
 (segment (start 94.5 75.5) (end 96 77) (width 0.2) (layer "F.Cu") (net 1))
 (segment (start 99.5 70.045) (end 99.5 65.5) (width 0.2) (layer "F.Cu") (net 4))
 (segment (start 99.5 65.5) (end 129 65.5) (width 0.2) (layer "F.Cu") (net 4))
 (segment (start 132.128 68.048) (end 132.75 68.67) (width 0.2) (layer "F.Cu") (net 4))
 (segment (start 129 65.5) (end 131.548 68.048) (width 0.2) (layer "F.Cu") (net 4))
 (segment (start 131.548 68.048) (end 132.128 68.048) (width 0.2) (layer "F.Cu") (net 4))
 (segment (start 98.26625 71.27875) (end 99.5 70.045) (width 0.2) (layer "F.Cu") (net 4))
 (segment (start 127.79 66.25) (end 132.75 71.21) (width 0.2) (layer "F.Cu") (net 6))
 (segment (start 117.31625 71.27875) (end 122.345 66.25) (width 0.2) (layer "F.Cu") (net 6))
 (segment (start 122.345 66.25) (end 127.79 66.25) (width 0.2) (layer "F.Cu") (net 6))
 (segment (start 131.128 73.128) (end 133.048 73.128) (width 0.2) (layer "F.Cu") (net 2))
 (segment (start 87.25 88.75) (end 102 88.75) (width 0.2) (layer "F.Cu") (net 2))
 (segment (start 116 88.5) (end 121.5 88.5) (width 0.2) (layer "F.Cu") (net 2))
 (segment (start 125.25 78.75) (end 130.872 73.128) (width 0.2) (layer "F.Cu") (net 2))
 (segment (start 125.25 89.6829) (end 125.25 78.75) (width 0.2) (layer "F.Cu") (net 2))
 (segment (start 125.21715 89.71575) (end 125.25 89.6829) (width 0.2) (layer "F.Cu") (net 2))
 (segment (start 102 88.75) (end 102.75 89.5) (width 0.2) (layer "F.Cu") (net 2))
 (segment (start 121.5 88.5) (end 122.71575 89.71575) (width 0.2) (layer "F.Cu") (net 2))
 (segment (start 130.872 73.128) (end 131.128 73.128) (width 0.2) (layer "F.Cu") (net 2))
 (segment (start 122.71575 89.71575) (end 125.21715 89.71575) (width 0.2) (layer "F.Cu") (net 2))
 (segment (start 102.75 89.5) (end 115 89.5) (width 0.2) (layer "F.Cu") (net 2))
 (segment (start 79.21625 90.32875) (end 79.25 90.295) (width 0.2) (layer "F.Cu") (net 2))
 (segment (start 85.67125 90.32875) (end 87.25 88.75) (width 0.2) (layer "F.Cu") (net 2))
 (segment (start 79.21625 90.32875) (end 85.67125 90.32875) (width 0.2) (layer "F.Cu") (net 2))
 (segment (start 115 89.5) (end 116 88.5) (width 0.2) (layer "F.Cu") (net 2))
 (segment (start 79.25 90.295) (end 79.25 90) (width 0.2) (layer "F.Cu") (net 2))
 (segment (start 130.71 76.29) (end 132.75 76.29) (width 0.2) (layer "F.Cu") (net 9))
 (segment (start 125.38325 90.11675) (end 128.5 87) (width 0.2) (layer "F.Cu") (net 9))
 (segment (start 117.52825 90.11675) (end 125.38325 90.11675) (width 0.2) (layer "F.Cu") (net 9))
 (segment (start 128.5 87) (end 128.5 78.5) (width 0.2) (layer "F.Cu") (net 9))
 (segment (start 117.31625 90.32875) (end 117.52825 90.11675) (width 0.2) (layer "F.Cu") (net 9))
 (segment (start 128.5 78.5) (end 130.71 76.29) (width 0.2) (layer "F.Cu") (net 9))
 (segment (start 116.75 95.75) (end 114 93) (width 0.2) (layer "F.Cu") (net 3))
 (segment (start 114 93) (end 114 90.32875) (width 0.2) (layer "F.Cu") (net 3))
 (segment (start 98.26625 90.32875) (end 114 90.32875) (width 0.2) (layer "F.Cu") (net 3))
 (segment (start 128.901 81.099) (end 128.901 89.099) (width 0.2) (layer "F.Cu") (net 3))
 (segment (start 132.75 78.83) (end 131.17 78.83) (width 0.2) (layer "F.Cu") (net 3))
 (segment (start 126.75 91.25) (end 125 91.25) (width 0.2) (layer "F.Cu") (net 3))
 (segment (start 122.25 95.75) (end 116.75 95.75) (width 0.2) (layer "F.Cu") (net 3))
 (segment (start 125 91.25) (end 124 92.25) (width 0.2) (layer "F.Cu") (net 3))
 (segment (start 131.17 78.83) (end 128.901 81.099) (width 0.2) (layer "F.Cu") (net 3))
 (segment (start 124 92.25) (end 124 94) (width 0.2) (layer "F.Cu") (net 3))
 (segment (start 124 94) (end 122.25 95.75) (width 0.2) (layer "F.Cu") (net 3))
 (segment (start 128.901 89.099) (end 126.75 91.25) (width 0.2) (layer "F.Cu") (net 3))
 (segment (start 132.99375 90.36875) (end 132.99375 81.61375) (width 0.2) (layer "F.Cu") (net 7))
 (segment (start 132.99375 81.61375) (end 132.75 81.37) (width 0.2) (layer "F.Cu") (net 7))
 (segment (start 140.13125 95.36875) (end 148.915 86.585) (width 0.2) (layer "F.Cu") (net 8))
 (segment (start 148.915 86.585) (end 148.915 81.37) (width 0.2) (layer "F.Cu") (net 8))
 (segment (start 132.99375 95.36875) (end 140.13125 95.36875) (width 0.2) (layer "F.Cu") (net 8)))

